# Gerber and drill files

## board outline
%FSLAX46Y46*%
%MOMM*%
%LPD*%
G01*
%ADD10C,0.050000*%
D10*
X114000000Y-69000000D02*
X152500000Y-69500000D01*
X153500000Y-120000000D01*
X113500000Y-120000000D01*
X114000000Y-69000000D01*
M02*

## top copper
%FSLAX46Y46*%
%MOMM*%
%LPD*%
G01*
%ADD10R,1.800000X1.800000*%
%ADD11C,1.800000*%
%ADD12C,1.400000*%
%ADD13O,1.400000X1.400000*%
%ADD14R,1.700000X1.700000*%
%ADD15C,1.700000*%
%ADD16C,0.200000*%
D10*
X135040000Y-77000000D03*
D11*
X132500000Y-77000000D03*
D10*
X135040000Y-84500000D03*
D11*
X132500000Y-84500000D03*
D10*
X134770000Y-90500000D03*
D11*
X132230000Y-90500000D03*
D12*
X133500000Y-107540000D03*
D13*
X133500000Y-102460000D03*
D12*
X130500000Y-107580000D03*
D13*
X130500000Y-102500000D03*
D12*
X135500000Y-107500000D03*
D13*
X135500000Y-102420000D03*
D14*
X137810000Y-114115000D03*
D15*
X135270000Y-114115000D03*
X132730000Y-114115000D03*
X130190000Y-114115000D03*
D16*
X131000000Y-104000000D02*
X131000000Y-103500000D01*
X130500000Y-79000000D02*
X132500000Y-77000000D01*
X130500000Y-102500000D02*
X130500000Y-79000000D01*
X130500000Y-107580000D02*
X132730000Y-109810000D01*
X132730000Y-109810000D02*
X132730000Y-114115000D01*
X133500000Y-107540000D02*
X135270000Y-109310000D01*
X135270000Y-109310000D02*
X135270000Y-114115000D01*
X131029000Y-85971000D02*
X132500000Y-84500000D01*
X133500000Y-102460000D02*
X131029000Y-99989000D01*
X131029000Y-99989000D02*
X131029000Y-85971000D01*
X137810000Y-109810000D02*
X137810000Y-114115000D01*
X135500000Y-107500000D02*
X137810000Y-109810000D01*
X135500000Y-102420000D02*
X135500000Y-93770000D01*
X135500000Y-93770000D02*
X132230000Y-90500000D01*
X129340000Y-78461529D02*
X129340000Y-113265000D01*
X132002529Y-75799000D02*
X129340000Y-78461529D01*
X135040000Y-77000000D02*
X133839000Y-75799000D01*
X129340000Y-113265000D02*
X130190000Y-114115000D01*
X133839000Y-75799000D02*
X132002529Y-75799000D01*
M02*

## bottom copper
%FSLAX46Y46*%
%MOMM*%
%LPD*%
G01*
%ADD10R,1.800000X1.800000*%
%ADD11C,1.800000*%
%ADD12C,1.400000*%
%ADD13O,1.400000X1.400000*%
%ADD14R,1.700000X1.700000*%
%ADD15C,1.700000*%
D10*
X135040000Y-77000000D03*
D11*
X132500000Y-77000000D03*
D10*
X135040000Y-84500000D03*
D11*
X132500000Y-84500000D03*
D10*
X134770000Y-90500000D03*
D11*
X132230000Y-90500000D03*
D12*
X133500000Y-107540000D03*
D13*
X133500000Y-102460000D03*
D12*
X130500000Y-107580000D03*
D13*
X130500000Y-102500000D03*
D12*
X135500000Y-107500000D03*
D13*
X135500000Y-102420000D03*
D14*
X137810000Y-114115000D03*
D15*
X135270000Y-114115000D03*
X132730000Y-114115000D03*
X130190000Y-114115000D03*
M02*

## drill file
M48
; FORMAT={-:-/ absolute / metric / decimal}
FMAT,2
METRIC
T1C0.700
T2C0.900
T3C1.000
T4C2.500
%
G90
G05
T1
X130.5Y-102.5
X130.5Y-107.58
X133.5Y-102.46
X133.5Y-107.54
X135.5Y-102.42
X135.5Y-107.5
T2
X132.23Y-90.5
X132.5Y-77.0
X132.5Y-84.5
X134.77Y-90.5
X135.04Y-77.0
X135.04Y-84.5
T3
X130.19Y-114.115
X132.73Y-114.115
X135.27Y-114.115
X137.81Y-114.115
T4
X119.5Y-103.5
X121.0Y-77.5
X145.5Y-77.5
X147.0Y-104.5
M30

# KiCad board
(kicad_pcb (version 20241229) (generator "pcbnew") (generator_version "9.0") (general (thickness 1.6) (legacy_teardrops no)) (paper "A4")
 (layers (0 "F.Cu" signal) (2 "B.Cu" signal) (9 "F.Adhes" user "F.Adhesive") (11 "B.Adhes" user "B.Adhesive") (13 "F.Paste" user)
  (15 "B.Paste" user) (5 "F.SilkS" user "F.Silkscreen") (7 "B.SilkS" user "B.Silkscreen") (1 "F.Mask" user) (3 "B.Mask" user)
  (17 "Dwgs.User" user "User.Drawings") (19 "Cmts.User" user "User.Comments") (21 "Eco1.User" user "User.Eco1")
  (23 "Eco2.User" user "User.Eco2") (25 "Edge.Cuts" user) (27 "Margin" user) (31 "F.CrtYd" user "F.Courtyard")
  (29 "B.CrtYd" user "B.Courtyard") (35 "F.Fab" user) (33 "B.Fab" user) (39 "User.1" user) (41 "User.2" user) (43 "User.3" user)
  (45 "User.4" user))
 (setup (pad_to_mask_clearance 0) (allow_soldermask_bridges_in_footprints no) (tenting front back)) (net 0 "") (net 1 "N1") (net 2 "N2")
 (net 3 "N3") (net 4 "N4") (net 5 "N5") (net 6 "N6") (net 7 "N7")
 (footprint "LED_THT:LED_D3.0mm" (layer "F.Cu") (at 135.04 77 180)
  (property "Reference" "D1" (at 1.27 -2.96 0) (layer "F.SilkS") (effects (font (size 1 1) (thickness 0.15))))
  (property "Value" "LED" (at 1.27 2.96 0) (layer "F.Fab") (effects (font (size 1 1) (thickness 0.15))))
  (pad "1" thru_hole rect (at 0 0 180) (size 1.8 1.8) (drill 0.9) (layers "*.Cu" "*.Mask") (remove_unused_layers no) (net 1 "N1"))
  (pad "2" thru_hole circle (at 2.54 0 180) (size 1.8 1.8) (drill 0.9) (layers "*.Cu" "*.Mask") (remove_unused_layers no) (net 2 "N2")))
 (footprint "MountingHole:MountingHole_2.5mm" (layer "F.Cu") (at 121 77.5)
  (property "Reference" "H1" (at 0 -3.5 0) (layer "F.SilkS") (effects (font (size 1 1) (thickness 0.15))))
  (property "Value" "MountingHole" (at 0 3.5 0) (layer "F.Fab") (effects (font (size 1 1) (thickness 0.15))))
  (pad "" np_thru_hole circle (at 0 0) (size 2.5 2.5) (drill 2.5) (layers "*.Cu" "*.Mask")))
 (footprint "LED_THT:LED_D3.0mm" (layer "F.Cu") (at 135.04 84.5 180)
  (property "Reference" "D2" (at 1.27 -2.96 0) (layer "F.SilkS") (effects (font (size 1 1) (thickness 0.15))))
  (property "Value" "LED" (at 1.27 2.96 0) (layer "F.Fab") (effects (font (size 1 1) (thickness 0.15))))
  (pad "1" thru_hole rect (at 0 0 180) (size 1.8 1.8) (drill 0.9) (layers "*.Cu" "*.Mask") (remove_unused_layers no) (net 1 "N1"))
  (pad "2" thru_hole circle (at 2.54 0 180) (size 1.8 1.8) (drill 0.9) (layers "*.Cu" "*.Mask") (remove_unused_layers no) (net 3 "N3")))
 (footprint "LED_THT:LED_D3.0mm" (layer "F.Cu") (at 134.77 90.5 180)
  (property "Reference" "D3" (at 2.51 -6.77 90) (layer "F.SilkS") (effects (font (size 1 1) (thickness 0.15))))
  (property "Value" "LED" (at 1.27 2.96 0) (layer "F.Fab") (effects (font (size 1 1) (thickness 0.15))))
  (pad "1" thru_hole rect (at 0 0 180) (size 1.8 1.8) (drill 0.9) (layers "*.Cu" "*.Mask") (remove_unused_layers no) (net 1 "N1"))
  (pad "2" thru_hole circle (at 2.54 0 180) (size 1.8 1.8) (drill 0.9) (layers "*.Cu" "*.Mask") (remove_unused_layers no) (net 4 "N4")))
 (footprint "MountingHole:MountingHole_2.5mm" (layer "F.Cu") (at 147 104.5)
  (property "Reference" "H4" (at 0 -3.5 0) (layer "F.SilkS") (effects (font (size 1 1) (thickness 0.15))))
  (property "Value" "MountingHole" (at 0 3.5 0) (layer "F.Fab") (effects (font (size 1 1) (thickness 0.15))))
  (pad "" np_thru_hole circle (at 0 0) (size 2.5 2.5) (drill 2.5) (layers "*.Cu" "*.Mask")))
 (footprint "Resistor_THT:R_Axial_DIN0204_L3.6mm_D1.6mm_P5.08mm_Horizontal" (layer "F.Cu") (at 133.5 107.54 90)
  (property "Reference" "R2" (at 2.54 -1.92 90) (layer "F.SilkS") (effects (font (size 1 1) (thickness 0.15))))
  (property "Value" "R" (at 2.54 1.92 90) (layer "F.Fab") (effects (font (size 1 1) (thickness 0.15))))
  (pad "1" thru_hole circle (at 0 0 90) (size 1.4 1.4) (drill 0.7) (layers "*.Cu" "*.Mask") (remove_unused_layers no) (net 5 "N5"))
  (pad "2" thru_hole oval (at 5.08 0 90) (size 1.4 1.4) (drill 0.7) (layers "*.Cu" "*.Mask") (remove_unused_layers no) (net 3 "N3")))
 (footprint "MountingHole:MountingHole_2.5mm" (layer "F.Cu") (at 145.5 77.5)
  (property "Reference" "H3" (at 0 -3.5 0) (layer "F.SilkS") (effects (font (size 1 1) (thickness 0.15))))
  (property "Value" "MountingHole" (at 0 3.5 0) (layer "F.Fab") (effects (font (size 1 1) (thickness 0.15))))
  (pad "" np_thru_hole circle (at 0 0) (size 2.5 2.5) (drill 2.5) (layers "*.Cu" "*.Mask")))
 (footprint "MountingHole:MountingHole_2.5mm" (layer "F.Cu") (at 119.5 103.5)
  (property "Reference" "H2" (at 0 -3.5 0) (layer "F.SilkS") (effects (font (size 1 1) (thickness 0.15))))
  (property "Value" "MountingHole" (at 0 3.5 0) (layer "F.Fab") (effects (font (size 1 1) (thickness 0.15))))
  (pad "" np_thru_hole circle (at 0 0) (size 2.5 2.5) (drill 2.5) (layers "*.Cu" "*.Mask")))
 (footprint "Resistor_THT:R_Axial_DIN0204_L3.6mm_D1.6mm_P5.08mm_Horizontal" (layer "F.Cu") (at 130.5 107.58 90)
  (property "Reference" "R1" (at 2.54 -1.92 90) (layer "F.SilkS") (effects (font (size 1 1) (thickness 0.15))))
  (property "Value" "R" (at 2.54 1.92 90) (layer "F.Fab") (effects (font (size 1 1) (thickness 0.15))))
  (pad "1" thru_hole circle (at 0 0 90) (size 1.4 1.4) (drill 0.7) (layers "*.Cu" "*.Mask") (remove_unused_layers no) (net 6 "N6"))
  (pad "2" thru_hole oval (at 5.08 0 90) (size 1.4 1.4) (drill 0.7) (layers "*.Cu" "*.Mask") (remove_unused_layers no) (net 2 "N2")))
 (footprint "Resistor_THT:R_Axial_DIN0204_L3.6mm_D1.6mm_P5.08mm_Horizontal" (layer "F.Cu") (at 135.5 107.5 90)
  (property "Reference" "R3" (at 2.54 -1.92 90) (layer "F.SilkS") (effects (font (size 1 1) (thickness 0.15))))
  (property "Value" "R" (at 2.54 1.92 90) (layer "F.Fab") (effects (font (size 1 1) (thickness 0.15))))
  (pad "1" thru_hole circle (at 0 0 90) (size 1.4 1.4) (drill 0.7) (layers "*.Cu" "*.Mask") (remove_unused_layers no) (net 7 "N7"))
  (pad "2" thru_hole oval (at 5.08 0 90) (size 1.4 1.4) (drill 0.7) (layers "*.Cu" "*.Mask") (remove_unused_layers no) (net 4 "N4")))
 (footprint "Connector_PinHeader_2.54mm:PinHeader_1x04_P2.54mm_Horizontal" (layer "F.Cu") (at 137.81 114.115 -90)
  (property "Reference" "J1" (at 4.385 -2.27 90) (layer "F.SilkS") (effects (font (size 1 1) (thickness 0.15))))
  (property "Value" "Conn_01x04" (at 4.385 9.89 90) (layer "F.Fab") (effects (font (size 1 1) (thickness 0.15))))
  (pad "1" thru_hole rect (at 0 0 270) (size 1.7 1.7) (drill 1) (layers "*.Cu" "*.Mask") (remove_unused_layers no) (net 7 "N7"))
  (pad "2" thru_hole circle (at 0 2.54 270) (size 1.7 1.7) (drill 1) (layers "*.Cu" "*.Mask") (remove_unused_layers no) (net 5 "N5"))
  (pad "3" thru_hole circle (at 0 5.08 270) (size 1.7 1.7) (drill 1) (layers "*.Cu" "*.Mask") (remove_unused_layers no) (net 6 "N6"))
  (pad "4" thru_hole circle (at 0 7.62 270) (size 1.7 1.7) (drill 1) (layers "*.Cu" "*.Mask") (remove_unused_layers no) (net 1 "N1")))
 (gr_poly (pts (xy 114 69) (xy 152.5 69.5) (xy 153.5 120) (xy 113.5 120)) (stroke (width 0.05) (type solid)) (fill no) (layer "Edge.Cuts"))
 (segment (start 131 104) (end 131 103.5) (width 0.2) (layer "F.Cu") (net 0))
 (segment (start 130.5 79) (end 132.5 77) (width 0.2) (layer "F.Cu") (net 2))
 (segment (start 130.5 102.5) (end 130.5 79) (width 0.2) (layer "F.Cu") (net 2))
 (segment (start 130.5 107.58) (end 132.73 109.81) (width 0.2) (layer "F.Cu") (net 6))
 (segment (start 132.73 109.81) (end 132.73 114.115) (width 0.2) (layer "F.Cu") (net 6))
 (segment (start 133.5 107.54) (end 135.27 109.31) (width 0.2) (layer "F.Cu") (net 5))
 (segment (start 135.27 109.31) (end 135.27 114.115) (width 0.2) (layer "F.Cu") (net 5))
 (segment (start 131.029 85.971) (end 132.5 84.5) (width 0.2) (layer "F.Cu") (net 3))
 (segment (start 133.5 102.46) (end 131.029 99.989) (width 0.2) (layer "F.Cu") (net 3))
 (segment (start 131.029 99.989) (end 131.029 85.971) (width 0.2) (layer "F.Cu") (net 3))
 (segment (start 137.81 109.81) (end 137.81 114.115) (width 0.2) (layer "F.Cu") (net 7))
 (segment (start 135.5 107.5) (end 137.81 109.81) (width 0.2) (layer "F.Cu") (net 7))
 (segment (start 135.5 102.42) (end 135.5 93.77) (width 0.2) (layer "F.Cu") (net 4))
 (segment (start 135.5 93.77) (end 132.23 90.5) (width 0.2) (layer "F.Cu") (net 4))
 (segment (start 129.34 78.461529) (end 129.34 113.265) (width 0.2) (layer "F.Cu") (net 1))
 (segment (start 132.002529 75.799) (end 129.34 78.461529) (width 0.2) (layer "F.Cu") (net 1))
 (segment (start 135.04 77) (end 133.839 75.799) (width 0.2) (layer "F.Cu") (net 1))
 (segment (start 129.34 113.265) (end 130.19 114.115) (width 0.2) (layer "F.Cu") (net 1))
 (segment (start 133.839 75.799) (end 132.002529 75.799) (width 0.2) (layer "F.Cu") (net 1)))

